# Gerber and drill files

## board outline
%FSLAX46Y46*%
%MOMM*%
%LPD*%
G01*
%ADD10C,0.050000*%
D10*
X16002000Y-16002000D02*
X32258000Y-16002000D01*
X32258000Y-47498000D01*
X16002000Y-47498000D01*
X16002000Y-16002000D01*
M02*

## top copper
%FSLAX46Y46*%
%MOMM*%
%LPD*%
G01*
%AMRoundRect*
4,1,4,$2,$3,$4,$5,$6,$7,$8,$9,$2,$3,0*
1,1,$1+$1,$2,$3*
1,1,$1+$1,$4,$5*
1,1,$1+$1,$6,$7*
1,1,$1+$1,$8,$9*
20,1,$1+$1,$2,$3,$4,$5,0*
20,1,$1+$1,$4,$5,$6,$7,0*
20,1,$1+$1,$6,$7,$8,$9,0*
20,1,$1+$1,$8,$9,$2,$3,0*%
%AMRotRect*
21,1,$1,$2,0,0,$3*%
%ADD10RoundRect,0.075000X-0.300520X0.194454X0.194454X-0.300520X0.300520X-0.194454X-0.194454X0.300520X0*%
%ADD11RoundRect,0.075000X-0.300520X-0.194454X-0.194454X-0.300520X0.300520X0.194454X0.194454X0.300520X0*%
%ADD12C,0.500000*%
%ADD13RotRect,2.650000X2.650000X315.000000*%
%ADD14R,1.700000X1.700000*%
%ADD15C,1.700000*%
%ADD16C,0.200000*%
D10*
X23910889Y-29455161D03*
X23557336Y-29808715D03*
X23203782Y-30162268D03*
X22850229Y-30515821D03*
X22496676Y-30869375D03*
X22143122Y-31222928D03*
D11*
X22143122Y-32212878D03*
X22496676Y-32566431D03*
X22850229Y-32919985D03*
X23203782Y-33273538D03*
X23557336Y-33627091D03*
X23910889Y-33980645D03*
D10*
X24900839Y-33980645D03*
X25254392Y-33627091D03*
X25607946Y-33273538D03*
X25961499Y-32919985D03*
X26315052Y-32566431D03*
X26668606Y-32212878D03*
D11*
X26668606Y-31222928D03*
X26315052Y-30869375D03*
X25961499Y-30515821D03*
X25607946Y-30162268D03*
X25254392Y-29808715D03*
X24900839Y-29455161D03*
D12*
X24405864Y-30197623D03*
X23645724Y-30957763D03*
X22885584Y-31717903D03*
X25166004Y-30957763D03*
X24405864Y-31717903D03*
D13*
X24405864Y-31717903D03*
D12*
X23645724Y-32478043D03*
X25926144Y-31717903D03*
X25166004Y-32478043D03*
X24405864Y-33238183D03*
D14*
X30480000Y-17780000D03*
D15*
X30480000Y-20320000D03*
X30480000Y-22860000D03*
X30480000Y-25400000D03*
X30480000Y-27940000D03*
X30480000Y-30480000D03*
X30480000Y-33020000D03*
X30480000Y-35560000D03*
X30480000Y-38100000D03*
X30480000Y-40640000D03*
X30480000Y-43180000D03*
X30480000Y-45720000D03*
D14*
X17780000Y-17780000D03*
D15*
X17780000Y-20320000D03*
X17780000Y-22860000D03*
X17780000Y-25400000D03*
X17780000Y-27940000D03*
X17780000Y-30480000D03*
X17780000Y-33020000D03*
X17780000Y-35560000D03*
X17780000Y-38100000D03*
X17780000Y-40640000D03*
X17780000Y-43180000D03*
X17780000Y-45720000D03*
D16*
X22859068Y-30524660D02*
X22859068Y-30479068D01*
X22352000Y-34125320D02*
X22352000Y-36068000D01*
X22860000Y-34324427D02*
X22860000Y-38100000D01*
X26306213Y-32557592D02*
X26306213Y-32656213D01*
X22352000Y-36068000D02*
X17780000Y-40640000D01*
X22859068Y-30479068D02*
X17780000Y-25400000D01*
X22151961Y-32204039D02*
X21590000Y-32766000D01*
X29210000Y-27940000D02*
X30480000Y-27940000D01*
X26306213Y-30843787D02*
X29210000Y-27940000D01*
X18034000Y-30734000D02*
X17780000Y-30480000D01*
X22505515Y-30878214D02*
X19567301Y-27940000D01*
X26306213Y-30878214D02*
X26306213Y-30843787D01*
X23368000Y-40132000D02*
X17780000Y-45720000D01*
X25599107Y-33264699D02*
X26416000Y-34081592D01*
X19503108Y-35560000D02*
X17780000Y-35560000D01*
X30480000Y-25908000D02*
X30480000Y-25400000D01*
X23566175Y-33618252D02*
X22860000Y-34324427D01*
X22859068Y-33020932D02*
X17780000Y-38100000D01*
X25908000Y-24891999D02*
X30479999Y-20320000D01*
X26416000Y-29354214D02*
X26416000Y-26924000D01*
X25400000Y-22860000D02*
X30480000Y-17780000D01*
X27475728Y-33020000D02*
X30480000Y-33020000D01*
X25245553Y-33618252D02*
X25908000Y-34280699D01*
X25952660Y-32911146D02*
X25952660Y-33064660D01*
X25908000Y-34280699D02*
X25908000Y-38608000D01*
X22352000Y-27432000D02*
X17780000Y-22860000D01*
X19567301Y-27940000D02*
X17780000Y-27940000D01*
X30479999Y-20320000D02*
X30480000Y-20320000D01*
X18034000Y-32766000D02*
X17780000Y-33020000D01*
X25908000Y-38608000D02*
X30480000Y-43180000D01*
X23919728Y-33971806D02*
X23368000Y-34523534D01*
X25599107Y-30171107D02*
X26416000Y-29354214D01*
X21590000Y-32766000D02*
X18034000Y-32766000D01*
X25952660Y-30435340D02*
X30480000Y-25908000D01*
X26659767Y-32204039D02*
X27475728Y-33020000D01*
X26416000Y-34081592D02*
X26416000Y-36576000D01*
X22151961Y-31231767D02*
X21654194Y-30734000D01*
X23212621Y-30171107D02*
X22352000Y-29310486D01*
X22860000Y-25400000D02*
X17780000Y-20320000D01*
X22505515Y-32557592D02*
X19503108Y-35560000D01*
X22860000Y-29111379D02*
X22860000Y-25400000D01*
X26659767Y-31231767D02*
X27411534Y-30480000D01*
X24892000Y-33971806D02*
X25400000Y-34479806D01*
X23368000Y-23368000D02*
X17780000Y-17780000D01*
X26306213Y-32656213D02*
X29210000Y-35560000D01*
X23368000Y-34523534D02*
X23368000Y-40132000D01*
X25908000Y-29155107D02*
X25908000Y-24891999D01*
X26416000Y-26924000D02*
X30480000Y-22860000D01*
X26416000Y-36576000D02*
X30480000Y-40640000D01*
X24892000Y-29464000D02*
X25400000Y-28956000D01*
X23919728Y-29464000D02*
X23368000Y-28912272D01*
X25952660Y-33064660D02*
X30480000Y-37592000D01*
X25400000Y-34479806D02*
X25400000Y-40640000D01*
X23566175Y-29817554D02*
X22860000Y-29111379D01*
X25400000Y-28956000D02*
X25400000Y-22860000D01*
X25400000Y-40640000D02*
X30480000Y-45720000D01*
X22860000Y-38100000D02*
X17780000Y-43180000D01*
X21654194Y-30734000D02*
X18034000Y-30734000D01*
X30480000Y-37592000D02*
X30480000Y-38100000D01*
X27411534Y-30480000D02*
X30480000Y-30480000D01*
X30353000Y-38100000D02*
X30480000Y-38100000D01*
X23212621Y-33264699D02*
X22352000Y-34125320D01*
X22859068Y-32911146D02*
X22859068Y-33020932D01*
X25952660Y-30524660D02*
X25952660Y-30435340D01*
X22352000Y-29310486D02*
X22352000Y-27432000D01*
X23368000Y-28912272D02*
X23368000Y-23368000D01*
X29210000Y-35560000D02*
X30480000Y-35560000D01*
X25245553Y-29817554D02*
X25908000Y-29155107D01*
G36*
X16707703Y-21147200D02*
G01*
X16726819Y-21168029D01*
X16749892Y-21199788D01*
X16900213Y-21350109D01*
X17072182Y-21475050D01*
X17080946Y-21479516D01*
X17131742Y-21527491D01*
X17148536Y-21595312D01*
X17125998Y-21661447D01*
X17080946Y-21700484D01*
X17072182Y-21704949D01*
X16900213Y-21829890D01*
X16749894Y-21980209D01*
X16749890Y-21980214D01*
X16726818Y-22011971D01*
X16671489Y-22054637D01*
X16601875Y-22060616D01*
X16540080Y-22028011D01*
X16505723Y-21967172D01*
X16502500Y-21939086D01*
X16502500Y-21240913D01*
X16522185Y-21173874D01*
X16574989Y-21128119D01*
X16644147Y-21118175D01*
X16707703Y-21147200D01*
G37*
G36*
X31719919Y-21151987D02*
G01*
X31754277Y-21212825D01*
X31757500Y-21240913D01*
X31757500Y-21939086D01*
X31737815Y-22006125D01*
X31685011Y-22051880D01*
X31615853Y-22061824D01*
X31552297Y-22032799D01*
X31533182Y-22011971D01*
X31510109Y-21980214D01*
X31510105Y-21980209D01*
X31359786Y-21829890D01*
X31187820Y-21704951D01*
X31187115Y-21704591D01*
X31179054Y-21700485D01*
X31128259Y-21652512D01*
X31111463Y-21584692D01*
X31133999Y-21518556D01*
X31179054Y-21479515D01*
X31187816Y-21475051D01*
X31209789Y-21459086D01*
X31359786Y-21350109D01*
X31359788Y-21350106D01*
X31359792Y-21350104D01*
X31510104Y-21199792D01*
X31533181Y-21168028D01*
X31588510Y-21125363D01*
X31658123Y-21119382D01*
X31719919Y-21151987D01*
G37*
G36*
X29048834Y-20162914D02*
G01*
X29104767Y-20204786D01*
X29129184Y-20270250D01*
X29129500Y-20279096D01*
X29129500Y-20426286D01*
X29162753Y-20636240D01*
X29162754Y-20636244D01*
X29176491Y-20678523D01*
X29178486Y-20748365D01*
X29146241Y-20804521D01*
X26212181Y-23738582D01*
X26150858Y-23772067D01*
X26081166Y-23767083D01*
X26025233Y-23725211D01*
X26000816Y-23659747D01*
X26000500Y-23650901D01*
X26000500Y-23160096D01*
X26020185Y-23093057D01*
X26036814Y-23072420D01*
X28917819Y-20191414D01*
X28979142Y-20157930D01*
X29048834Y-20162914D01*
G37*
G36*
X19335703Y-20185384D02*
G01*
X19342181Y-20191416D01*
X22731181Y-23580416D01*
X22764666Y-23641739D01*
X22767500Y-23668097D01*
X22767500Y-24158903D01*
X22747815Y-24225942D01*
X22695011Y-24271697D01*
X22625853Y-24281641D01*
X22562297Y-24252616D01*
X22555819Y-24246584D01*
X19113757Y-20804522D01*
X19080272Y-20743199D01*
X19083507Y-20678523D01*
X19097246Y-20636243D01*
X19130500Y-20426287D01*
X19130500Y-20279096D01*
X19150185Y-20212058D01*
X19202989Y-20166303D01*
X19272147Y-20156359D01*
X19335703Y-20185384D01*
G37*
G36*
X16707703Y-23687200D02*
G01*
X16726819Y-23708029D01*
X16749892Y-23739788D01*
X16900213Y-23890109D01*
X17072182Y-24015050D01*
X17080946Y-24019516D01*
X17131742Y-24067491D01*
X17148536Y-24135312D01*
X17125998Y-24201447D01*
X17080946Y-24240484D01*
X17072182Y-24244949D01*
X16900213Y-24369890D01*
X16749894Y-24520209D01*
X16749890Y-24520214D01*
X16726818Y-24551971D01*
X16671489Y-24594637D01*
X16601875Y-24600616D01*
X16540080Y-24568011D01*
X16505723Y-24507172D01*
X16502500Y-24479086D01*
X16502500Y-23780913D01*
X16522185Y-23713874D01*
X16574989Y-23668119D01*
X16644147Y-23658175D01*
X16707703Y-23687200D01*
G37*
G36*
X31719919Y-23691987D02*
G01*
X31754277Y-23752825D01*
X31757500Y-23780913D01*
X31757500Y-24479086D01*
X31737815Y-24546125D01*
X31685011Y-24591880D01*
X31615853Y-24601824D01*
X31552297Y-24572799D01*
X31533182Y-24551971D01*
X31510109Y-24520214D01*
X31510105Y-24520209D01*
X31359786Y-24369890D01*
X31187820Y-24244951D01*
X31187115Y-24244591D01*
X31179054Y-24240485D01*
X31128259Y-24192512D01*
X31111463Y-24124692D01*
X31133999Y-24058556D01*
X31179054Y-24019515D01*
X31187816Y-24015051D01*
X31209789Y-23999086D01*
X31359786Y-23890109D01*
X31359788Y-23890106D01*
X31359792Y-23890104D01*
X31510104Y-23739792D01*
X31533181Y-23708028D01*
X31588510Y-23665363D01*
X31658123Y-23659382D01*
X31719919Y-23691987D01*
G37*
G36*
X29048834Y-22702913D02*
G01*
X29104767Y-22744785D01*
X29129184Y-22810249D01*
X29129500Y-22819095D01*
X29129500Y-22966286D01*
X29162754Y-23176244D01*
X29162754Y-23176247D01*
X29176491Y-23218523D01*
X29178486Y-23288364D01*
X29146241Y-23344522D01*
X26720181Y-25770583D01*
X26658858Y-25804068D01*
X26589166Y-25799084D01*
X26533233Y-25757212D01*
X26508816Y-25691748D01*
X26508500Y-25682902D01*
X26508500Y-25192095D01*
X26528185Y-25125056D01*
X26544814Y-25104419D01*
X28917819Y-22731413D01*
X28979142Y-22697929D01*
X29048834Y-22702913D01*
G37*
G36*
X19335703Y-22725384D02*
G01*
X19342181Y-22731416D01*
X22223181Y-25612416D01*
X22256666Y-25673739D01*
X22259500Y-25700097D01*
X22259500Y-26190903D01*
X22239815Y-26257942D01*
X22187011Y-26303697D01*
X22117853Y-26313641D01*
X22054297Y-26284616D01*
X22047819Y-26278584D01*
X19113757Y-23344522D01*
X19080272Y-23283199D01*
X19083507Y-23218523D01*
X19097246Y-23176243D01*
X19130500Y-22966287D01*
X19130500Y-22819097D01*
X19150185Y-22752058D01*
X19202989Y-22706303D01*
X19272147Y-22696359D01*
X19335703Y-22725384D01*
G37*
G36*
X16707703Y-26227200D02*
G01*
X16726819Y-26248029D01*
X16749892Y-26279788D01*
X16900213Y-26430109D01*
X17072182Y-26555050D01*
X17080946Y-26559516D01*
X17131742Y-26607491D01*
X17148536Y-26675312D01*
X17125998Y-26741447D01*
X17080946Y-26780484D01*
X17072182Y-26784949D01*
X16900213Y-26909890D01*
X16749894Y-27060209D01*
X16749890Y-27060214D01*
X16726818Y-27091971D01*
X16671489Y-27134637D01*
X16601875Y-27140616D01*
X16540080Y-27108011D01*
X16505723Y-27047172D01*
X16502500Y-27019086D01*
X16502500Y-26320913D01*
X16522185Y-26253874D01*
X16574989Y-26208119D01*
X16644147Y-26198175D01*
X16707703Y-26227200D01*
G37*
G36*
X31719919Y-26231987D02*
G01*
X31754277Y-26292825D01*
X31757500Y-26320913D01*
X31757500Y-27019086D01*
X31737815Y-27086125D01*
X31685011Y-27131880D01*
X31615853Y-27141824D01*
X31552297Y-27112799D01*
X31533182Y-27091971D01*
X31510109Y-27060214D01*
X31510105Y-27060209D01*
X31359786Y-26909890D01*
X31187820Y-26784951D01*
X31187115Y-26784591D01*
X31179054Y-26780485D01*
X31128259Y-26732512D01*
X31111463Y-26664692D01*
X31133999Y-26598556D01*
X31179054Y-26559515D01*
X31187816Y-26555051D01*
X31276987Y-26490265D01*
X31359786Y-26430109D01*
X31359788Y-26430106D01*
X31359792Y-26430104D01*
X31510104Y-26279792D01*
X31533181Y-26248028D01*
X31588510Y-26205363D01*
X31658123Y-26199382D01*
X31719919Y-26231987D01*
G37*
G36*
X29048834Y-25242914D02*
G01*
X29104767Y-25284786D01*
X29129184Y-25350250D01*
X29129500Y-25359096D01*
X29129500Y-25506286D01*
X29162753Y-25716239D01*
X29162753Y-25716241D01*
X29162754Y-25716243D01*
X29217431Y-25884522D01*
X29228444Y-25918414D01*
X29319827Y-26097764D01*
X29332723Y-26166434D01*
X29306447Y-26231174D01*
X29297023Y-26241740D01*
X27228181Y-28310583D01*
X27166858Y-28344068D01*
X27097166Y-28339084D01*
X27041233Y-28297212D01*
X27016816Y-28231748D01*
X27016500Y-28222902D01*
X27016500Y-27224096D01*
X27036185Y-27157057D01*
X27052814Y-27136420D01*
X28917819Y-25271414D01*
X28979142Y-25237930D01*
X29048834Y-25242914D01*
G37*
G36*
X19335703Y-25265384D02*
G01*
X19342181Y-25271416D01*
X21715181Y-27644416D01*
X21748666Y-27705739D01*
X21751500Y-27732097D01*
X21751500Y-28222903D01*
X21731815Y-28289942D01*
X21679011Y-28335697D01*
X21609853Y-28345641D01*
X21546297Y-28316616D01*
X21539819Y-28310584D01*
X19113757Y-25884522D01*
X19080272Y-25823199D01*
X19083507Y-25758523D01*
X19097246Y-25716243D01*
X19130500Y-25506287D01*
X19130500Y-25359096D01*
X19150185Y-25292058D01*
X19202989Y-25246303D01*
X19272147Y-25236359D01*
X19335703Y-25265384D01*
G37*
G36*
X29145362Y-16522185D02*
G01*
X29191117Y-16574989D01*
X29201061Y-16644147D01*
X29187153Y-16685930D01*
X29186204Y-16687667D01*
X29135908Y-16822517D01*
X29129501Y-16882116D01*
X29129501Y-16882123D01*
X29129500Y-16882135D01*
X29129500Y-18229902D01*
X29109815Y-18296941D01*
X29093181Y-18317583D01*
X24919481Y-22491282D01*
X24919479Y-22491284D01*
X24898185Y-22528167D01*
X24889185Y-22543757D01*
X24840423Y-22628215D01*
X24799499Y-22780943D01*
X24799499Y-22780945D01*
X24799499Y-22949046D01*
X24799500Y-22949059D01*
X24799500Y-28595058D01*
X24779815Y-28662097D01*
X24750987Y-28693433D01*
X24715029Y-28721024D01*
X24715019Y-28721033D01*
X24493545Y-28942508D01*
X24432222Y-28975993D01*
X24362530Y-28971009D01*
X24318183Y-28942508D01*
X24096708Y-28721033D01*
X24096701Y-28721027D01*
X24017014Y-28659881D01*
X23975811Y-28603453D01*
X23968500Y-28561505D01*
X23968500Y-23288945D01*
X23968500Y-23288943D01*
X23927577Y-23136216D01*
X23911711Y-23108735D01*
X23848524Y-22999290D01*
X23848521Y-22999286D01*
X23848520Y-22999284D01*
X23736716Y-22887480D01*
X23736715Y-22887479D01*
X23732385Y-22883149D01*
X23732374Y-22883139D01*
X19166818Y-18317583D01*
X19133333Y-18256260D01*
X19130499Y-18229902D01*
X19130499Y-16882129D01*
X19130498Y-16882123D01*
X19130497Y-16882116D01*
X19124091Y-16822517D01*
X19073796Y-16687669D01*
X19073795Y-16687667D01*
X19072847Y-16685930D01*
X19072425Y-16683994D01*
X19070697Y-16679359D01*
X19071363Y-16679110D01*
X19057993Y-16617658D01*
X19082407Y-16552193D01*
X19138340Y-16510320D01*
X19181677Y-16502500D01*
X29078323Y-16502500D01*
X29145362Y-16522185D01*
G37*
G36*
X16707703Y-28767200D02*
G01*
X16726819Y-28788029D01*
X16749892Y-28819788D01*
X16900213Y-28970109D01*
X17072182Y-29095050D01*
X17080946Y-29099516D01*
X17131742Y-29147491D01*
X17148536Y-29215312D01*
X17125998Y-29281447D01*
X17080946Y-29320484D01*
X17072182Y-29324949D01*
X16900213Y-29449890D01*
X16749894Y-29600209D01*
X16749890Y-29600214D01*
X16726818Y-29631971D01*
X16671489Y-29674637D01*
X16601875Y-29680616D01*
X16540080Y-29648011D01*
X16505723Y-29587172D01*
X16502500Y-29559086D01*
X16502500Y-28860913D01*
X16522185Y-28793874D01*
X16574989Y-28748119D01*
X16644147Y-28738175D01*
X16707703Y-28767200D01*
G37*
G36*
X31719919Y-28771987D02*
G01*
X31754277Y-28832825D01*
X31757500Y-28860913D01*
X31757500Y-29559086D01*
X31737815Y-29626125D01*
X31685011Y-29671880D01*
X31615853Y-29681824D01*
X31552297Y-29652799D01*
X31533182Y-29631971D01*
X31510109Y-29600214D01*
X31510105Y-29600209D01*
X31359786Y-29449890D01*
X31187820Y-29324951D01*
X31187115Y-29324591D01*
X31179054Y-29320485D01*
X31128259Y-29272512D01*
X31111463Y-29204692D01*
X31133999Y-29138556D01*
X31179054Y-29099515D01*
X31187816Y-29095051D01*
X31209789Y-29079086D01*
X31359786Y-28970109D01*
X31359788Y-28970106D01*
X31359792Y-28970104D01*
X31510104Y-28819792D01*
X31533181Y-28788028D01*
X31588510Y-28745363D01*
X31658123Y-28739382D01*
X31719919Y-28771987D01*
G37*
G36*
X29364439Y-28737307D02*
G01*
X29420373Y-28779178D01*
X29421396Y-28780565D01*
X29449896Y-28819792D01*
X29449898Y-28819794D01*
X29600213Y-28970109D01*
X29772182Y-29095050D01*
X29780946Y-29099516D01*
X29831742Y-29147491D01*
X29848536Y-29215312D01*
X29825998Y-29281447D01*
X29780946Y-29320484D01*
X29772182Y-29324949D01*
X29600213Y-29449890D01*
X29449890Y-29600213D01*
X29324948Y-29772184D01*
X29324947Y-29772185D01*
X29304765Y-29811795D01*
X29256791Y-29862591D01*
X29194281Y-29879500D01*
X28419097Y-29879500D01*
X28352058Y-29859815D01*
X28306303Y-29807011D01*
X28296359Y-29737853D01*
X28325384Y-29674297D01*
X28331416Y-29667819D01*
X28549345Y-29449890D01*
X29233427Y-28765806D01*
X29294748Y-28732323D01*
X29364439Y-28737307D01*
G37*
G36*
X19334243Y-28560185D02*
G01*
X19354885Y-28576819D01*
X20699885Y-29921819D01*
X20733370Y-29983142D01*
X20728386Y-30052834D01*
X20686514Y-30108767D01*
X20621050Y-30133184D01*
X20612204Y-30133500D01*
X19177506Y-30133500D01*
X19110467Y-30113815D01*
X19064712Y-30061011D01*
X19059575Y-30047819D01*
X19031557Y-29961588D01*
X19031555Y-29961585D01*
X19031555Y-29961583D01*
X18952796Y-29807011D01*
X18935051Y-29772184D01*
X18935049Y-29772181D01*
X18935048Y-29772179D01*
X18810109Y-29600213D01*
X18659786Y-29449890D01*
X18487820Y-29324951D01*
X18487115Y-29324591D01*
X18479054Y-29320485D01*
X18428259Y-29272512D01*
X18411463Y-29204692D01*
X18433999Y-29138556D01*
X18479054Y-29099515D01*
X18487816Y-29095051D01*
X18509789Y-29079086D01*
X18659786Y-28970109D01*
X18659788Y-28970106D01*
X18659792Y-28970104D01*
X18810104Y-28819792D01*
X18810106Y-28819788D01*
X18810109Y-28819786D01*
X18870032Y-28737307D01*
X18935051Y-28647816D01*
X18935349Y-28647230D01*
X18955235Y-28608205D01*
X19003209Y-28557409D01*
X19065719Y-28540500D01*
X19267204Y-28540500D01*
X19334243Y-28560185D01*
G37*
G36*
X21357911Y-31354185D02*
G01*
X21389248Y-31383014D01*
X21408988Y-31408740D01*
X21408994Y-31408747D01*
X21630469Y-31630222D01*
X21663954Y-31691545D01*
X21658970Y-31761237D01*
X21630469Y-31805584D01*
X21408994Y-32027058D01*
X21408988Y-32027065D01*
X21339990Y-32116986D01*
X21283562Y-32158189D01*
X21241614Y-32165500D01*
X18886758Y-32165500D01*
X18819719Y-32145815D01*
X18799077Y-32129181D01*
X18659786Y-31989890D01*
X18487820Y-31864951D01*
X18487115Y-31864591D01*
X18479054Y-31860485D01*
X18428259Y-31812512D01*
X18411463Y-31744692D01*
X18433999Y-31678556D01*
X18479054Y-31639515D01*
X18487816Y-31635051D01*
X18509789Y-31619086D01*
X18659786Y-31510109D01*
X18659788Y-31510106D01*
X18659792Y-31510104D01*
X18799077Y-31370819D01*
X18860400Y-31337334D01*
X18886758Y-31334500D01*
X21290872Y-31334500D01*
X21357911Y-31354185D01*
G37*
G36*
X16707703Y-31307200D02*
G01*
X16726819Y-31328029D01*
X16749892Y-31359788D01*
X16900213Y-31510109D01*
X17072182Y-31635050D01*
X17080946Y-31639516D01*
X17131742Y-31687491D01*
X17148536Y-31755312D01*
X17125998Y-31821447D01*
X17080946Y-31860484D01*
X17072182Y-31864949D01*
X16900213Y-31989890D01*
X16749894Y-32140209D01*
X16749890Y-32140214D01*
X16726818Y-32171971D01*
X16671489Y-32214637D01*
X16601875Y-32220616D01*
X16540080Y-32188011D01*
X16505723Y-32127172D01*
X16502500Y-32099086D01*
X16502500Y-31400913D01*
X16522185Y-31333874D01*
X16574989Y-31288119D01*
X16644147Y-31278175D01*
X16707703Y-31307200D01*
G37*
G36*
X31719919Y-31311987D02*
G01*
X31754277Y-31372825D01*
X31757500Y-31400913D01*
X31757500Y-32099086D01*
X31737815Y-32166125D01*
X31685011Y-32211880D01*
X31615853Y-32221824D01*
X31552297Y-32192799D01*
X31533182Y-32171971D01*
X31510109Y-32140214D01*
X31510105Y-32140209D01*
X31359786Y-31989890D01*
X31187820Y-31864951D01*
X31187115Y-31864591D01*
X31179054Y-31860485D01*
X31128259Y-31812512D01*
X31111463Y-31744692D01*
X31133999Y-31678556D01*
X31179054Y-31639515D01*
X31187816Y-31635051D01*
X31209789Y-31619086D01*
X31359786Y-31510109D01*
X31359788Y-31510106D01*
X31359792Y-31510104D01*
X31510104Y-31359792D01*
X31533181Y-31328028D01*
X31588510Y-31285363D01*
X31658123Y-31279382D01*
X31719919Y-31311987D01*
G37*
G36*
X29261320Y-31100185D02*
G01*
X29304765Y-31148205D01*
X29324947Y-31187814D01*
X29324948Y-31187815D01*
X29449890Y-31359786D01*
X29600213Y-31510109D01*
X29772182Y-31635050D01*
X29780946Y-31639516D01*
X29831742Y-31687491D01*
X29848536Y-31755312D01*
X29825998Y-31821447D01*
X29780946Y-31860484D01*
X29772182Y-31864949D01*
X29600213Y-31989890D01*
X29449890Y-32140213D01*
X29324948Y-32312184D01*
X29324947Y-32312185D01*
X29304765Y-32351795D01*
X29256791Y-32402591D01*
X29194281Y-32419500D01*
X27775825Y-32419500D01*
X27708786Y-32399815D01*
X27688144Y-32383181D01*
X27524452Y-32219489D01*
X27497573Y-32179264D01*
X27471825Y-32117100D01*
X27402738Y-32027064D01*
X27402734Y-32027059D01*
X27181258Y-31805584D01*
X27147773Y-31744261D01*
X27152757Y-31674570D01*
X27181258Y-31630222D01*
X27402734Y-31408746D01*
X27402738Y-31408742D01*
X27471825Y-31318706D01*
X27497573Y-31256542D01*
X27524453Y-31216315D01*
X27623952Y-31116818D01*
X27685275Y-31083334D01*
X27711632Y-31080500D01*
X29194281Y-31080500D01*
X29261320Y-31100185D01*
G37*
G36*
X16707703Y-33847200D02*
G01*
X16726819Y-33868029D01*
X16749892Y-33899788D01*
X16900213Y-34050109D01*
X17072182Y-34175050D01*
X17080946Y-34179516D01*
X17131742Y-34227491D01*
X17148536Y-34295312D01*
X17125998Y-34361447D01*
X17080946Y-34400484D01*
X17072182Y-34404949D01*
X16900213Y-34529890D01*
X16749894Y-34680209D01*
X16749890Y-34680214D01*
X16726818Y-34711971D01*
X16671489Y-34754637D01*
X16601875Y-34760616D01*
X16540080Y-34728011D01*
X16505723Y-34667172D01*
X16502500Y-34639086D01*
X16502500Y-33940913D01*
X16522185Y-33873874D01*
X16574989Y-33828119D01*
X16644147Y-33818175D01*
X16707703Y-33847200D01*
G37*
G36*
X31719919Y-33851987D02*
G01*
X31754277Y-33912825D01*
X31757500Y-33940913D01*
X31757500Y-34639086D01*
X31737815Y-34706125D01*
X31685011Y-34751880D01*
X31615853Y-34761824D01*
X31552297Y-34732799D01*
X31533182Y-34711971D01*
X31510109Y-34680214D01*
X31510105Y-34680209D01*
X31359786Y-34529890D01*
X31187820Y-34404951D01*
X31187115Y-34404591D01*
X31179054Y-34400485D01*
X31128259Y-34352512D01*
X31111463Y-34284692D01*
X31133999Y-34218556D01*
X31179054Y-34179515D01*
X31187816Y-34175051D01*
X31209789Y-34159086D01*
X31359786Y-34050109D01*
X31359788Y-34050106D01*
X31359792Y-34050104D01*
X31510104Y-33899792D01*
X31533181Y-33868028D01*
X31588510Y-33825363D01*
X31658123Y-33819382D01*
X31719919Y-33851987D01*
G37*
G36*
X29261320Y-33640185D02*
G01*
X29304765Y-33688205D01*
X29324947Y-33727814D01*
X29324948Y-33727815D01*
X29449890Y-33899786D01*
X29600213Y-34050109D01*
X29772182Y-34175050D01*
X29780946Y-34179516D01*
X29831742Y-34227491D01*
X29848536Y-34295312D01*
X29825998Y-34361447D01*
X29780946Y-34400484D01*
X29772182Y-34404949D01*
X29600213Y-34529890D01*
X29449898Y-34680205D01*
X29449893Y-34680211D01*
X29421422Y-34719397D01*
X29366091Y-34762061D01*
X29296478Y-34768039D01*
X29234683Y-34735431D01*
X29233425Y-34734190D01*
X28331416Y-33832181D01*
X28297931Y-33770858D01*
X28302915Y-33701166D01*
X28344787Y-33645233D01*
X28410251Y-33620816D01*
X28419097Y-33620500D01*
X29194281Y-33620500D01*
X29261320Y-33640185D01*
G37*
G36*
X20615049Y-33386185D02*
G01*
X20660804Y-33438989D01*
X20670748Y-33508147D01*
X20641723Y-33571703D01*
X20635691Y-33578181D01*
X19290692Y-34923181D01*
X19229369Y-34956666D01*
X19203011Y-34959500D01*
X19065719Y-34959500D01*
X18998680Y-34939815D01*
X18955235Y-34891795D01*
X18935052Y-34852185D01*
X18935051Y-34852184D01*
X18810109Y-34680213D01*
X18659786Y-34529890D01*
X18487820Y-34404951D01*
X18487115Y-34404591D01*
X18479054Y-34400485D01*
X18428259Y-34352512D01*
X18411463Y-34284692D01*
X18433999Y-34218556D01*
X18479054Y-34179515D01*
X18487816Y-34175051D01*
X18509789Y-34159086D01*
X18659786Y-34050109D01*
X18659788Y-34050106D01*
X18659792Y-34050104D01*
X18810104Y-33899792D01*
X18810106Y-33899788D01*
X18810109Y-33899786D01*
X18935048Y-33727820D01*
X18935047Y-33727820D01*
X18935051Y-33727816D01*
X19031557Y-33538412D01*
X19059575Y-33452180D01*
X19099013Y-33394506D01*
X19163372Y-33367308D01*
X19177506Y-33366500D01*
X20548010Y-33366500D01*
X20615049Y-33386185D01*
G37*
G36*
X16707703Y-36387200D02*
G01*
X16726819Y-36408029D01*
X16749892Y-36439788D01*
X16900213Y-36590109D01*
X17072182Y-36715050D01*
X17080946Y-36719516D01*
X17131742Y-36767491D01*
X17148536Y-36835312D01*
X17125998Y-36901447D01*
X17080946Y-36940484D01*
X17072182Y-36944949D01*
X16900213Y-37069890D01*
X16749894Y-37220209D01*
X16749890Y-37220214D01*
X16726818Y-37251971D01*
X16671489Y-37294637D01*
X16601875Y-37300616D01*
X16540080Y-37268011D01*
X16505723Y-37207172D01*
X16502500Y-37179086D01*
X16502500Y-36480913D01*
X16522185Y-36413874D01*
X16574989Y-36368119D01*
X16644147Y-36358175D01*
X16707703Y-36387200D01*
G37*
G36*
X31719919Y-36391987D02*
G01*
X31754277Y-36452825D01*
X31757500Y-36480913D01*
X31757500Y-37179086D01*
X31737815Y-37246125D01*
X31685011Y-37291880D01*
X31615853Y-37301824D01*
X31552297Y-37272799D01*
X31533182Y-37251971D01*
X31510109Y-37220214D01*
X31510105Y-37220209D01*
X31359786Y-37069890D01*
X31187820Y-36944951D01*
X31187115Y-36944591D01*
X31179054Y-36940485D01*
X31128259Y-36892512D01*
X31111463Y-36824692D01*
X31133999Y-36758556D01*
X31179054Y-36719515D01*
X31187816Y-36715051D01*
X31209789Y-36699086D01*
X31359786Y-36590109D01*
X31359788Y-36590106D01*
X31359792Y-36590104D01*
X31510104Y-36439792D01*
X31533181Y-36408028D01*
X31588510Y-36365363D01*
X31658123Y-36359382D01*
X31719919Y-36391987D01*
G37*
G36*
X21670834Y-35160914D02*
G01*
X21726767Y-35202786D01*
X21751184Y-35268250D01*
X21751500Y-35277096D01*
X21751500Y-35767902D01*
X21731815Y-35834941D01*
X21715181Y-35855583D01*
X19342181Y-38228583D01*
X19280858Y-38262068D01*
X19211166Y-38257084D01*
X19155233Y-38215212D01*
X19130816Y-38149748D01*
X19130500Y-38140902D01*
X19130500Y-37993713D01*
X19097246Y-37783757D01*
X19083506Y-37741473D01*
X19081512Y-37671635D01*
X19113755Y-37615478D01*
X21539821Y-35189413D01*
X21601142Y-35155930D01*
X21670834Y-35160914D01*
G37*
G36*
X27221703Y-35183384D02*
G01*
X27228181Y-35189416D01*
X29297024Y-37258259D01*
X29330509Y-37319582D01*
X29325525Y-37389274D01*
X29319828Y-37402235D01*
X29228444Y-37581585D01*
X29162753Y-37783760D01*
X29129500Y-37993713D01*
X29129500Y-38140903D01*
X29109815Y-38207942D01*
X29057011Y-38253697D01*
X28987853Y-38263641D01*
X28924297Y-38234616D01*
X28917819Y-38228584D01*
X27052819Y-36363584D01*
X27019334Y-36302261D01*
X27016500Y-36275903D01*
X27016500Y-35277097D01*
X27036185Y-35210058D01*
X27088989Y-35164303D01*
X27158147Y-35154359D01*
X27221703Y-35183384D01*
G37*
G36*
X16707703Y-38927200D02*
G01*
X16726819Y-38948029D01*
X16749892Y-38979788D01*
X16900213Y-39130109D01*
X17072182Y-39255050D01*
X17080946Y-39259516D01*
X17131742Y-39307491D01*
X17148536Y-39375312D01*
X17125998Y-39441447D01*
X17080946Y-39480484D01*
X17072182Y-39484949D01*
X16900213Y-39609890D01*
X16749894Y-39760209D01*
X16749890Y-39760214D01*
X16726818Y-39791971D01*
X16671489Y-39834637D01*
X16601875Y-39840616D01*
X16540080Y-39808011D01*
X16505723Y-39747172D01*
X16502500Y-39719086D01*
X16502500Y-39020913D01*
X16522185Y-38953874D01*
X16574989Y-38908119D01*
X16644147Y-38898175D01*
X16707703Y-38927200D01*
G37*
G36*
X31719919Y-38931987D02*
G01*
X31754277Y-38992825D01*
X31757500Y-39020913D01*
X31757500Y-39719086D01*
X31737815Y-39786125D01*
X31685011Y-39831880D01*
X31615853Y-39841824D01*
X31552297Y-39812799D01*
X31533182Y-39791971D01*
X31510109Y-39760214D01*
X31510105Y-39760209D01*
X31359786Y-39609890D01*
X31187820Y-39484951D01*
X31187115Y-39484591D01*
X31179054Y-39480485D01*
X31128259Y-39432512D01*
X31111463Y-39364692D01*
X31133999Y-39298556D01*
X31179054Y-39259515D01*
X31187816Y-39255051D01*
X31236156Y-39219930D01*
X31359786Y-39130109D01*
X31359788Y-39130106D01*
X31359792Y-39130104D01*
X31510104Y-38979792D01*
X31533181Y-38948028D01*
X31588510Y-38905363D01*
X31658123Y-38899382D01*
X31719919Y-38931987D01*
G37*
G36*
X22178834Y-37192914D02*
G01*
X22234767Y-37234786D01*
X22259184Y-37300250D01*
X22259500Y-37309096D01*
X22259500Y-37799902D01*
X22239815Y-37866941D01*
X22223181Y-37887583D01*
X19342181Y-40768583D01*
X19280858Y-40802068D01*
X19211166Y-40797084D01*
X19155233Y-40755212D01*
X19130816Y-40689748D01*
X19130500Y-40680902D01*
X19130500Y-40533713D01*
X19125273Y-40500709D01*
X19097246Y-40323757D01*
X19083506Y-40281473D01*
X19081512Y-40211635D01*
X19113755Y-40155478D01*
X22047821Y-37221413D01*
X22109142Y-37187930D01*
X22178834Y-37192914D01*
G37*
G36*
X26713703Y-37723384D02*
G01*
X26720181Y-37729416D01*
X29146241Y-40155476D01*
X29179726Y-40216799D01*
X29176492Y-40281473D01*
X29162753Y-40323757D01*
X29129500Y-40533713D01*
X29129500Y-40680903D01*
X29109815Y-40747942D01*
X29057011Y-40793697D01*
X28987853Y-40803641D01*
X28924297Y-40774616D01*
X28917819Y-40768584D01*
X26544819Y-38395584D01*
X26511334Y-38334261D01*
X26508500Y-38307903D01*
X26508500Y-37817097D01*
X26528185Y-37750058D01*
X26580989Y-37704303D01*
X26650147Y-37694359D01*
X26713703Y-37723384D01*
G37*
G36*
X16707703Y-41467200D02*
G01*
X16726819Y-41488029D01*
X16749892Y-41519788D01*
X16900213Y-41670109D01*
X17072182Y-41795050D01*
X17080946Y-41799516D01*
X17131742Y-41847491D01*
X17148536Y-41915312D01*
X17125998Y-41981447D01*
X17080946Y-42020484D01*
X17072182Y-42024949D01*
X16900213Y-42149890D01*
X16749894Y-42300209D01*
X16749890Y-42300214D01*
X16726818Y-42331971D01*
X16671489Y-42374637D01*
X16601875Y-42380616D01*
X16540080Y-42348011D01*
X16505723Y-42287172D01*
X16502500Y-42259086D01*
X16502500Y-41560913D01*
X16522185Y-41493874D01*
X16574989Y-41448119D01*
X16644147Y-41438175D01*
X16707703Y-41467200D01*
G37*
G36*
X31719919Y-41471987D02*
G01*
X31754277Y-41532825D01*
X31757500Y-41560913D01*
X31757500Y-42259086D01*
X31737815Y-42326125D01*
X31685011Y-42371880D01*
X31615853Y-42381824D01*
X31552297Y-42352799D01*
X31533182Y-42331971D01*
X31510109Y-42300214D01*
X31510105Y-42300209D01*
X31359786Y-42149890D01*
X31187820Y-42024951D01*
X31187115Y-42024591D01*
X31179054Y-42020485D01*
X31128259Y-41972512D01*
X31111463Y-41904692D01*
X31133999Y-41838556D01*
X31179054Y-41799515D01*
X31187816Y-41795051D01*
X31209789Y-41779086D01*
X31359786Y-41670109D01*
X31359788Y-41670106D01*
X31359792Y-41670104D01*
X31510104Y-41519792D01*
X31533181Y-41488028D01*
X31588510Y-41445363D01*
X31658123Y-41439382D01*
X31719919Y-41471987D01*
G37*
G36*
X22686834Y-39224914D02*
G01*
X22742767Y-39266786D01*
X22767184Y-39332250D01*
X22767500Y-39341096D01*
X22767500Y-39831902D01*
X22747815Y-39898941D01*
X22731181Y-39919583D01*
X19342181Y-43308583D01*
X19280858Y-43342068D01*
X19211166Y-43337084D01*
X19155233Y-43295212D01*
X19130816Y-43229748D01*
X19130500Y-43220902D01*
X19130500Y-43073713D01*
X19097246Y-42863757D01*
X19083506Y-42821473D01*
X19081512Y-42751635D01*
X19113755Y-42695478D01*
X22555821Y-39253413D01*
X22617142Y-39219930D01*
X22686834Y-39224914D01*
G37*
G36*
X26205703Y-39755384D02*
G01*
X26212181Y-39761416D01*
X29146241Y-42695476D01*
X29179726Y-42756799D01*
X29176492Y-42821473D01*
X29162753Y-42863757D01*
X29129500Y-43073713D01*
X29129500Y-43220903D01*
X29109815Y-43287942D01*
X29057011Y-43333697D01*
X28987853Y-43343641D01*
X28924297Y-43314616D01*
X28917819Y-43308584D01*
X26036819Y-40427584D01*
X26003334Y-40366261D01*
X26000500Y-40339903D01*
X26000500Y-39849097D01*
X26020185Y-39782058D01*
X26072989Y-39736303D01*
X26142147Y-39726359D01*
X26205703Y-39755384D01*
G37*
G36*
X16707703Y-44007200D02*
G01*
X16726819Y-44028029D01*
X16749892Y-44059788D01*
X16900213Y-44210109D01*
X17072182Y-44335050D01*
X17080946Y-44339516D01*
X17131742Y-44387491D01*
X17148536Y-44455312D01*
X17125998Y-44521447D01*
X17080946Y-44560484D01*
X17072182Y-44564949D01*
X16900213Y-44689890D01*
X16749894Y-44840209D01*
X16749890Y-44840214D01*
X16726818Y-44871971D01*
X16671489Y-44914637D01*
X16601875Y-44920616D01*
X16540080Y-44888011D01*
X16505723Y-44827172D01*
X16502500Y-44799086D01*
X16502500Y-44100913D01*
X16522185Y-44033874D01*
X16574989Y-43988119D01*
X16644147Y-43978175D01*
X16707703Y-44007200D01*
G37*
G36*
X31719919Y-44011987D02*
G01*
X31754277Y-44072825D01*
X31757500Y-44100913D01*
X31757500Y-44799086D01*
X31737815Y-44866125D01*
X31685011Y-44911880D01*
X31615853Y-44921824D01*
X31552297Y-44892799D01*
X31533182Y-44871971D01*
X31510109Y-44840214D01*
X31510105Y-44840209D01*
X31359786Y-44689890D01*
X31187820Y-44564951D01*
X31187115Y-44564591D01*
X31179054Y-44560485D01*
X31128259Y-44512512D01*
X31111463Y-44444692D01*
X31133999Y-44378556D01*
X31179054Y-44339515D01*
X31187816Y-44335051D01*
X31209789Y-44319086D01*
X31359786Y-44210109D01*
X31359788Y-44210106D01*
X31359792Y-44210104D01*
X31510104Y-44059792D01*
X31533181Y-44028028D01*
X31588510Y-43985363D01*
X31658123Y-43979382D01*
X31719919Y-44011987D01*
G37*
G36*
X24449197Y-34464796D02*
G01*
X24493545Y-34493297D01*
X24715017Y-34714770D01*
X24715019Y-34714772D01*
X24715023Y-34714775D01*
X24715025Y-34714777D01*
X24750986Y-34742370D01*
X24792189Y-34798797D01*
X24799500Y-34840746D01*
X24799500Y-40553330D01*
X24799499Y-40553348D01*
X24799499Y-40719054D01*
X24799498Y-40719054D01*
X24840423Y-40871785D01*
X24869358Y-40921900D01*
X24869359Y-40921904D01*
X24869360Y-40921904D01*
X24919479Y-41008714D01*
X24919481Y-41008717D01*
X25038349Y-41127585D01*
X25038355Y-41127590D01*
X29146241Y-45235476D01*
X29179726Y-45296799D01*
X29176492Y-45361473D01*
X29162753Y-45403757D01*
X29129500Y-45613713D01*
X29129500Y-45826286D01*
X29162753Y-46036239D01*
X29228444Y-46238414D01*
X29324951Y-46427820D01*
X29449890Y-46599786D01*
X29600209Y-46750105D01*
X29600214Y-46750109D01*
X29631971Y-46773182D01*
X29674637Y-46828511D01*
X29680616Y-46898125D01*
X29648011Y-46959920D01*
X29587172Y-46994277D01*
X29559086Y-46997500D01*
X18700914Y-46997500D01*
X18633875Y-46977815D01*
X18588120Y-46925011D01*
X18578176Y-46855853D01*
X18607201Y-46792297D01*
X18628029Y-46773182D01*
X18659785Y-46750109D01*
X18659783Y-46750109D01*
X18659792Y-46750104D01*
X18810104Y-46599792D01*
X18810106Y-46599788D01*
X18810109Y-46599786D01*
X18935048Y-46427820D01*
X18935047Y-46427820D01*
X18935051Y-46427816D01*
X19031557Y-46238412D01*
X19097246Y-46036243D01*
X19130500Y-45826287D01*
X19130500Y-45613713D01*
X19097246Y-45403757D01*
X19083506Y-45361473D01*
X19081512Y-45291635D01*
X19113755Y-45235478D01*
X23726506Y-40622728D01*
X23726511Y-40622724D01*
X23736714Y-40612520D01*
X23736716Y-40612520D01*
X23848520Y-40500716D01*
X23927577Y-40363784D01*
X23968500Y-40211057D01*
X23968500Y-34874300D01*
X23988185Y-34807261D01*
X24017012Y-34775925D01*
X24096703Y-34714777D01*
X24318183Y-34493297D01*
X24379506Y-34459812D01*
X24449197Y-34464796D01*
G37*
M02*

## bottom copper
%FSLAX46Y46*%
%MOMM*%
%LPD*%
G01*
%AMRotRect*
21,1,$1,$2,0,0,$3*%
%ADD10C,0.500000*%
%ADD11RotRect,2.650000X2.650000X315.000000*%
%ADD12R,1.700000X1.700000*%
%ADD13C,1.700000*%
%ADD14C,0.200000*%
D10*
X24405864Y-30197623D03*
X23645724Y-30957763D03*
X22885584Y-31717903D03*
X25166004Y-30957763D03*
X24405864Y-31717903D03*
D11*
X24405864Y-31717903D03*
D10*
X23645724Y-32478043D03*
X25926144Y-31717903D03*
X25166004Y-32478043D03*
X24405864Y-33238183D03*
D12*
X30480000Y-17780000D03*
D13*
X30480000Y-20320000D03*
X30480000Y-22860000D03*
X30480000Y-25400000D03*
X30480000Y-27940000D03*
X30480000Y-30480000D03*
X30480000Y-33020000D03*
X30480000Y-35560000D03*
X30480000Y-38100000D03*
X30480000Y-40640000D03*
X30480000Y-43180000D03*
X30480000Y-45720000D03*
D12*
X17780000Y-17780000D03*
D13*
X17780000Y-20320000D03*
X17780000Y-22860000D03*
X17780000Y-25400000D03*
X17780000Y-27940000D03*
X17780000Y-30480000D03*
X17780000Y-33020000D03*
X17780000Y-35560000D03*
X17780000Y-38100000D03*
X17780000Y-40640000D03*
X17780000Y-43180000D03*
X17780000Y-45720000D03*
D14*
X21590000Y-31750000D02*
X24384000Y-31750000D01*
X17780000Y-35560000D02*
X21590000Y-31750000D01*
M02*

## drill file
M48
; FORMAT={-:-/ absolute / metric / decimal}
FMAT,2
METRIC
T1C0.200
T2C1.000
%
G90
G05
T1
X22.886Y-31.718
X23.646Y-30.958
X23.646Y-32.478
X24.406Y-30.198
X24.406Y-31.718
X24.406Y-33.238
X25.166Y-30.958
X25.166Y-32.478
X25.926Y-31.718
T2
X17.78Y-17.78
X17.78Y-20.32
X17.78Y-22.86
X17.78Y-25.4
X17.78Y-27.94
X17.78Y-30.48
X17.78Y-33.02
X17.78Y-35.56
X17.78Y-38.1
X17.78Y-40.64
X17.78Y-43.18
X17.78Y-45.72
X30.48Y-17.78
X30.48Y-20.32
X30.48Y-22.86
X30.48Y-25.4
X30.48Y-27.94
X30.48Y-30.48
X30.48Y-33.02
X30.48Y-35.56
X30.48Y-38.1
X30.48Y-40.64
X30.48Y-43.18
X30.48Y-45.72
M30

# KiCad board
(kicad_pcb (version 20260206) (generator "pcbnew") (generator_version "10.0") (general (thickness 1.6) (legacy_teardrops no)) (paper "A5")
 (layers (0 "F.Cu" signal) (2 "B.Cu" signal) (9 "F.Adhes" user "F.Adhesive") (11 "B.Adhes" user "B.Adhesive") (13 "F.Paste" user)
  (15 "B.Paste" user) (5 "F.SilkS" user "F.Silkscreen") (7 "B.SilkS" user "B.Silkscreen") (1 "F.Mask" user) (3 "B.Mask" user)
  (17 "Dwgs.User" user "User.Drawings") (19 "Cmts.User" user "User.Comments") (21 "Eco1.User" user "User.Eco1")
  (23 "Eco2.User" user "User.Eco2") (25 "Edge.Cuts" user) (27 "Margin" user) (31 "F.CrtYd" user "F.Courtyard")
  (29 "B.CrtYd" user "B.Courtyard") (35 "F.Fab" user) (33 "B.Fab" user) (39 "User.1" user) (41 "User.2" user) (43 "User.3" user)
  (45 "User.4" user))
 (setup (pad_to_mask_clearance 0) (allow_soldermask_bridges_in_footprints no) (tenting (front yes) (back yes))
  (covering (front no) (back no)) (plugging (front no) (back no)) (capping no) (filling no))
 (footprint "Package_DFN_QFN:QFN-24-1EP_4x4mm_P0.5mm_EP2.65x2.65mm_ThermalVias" (layer "F.Cu") (at 24.405864 31.717903 -45)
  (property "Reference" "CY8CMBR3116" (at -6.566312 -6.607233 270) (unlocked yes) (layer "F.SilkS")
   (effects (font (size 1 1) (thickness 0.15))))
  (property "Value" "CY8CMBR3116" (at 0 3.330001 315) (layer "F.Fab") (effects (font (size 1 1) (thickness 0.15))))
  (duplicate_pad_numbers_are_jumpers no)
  (pad "" smd roundrect (at -0.66 -0.66 315) (size 1.15 1.15) (layers "F.Paste") (roundrect_rratio 0.217391))
  (pad "" smd roundrect (at -0.66 0.66 315) (size 1.15 1.15) (layers "F.Paste") (roundrect_rratio 0.217391))
  (pad "" smd roundrect (at 0.66 -0.66 315) (size 1.15 1.15) (layers "F.Paste") (roundrect_rratio 0.217391))
  (pad "" smd roundrect (at 0.66 0.66 315) (size 1.15 1.15) (layers "F.Paste") (roundrect_rratio 0.217391))
  (pad "1" smd roundrect (at -1.95 -1.25 315) (size 0.85 0.3) (layers "F.Cu" "F.Mask" "F.Paste") (roundrect_rratio 0.25) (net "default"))
  (pad "2" smd roundrect (at -1.95 -0.75 315) (size 0.85 0.3) (layers "F.Cu" "F.Mask" "F.Paste") (roundrect_rratio 0.25) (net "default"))
  (pad "3" smd roundrect (at -1.95 -0.25 315) (size 0.85 0.3) (layers "F.Cu" "F.Mask" "F.Paste") (roundrect_rratio 0.25) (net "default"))
  (pad "4" smd roundrect (at -1.95 0.25 315) (size 0.85 0.3) (layers "F.Cu" "F.Mask" "F.Paste") (roundrect_rratio 0.25) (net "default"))
  (pad "5" smd roundrect (at -1.95 0.75 315) (size 0.85 0.3) (layers "F.Cu" "F.Mask" "F.Paste") (roundrect_rratio 0.25) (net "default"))
  (pad "6" smd roundrect (at -1.95 1.25 315) (size 0.85 0.3) (layers "F.Cu" "F.Mask" "F.Paste") (roundrect_rratio 0.25) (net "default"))
  (pad "7" smd roundrect (at -1.25 1.95 315) (size 0.3 0.85) (layers "F.Cu" "F.Mask" "F.Paste") (roundrect_rratio 0.25) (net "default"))
  (pad "8" smd roundrect (at -0.75 1.95 315) (size 0.3 0.85) (layers "F.Cu" "F.Mask" "F.Paste") (roundrect_rratio 0.25) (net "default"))
  (pad "9" smd roundrect (at -0.25 1.95 315) (size 0.3 0.85) (layers "F.Cu" "F.Mask" "F.Paste") (roundrect_rratio 0.25) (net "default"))
  (pad "10" smd roundrect (at 0.25 1.95 315) (size 0.3 0.85) (layers "F.Cu" "F.Mask" "F.Paste") (roundrect_rratio 0.25) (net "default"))
  (pad "11" smd roundrect (at 0.75 1.95 315) (size 0.3 0.85) (layers "F.Cu" "F.Mask" "F.Paste") (roundrect_rratio 0.25) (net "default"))
  (pad "12" smd roundrect (at 1.25 1.95 315) (size 0.3 0.85) (layers "F.Cu" "F.Mask" "F.Paste") (roundrect_rratio 0.25) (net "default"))
  (pad "13" smd roundrect (at 1.95 1.25 315) (size 0.85 0.3) (layers "F.Cu" "F.Mask" "F.Paste") (roundrect_rratio 0.25) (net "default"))
  (pad "14" smd roundrect (at 1.95 0.75 315) (size 0.85 0.3) (layers "F.Cu" "F.Mask" "F.Paste") (roundrect_rratio 0.25) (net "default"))
  (pad "15" smd roundrect (at 1.95 0.25 315) (size 0.85 0.3) (layers "F.Cu" "F.Mask" "F.Paste") (roundrect_rratio 0.25) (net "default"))
  (pad "16" smd roundrect (at 1.95 -0.25 315) (size 0.85 0.3) (layers "F.Cu" "F.Mask" "F.Paste") (roundrect_rratio 0.25) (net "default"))
  (pad "17" smd roundrect (at 1.95 -0.75 315) (size 0.85 0.3) (layers "F.Cu" "F.Mask" "F.Paste") (roundrect_rratio 0.25) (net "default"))
  (pad "18" smd roundrect (at 1.95 -1.25 315) (size 0.85 0.3) (layers "F.Cu" "F.Mask" "F.Paste") (roundrect_rratio 0.25) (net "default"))
  (pad "19" smd roundrect (at 1.25 -1.95 315) (size 0.3 0.85) (layers "F.Cu" "F.Mask" "F.Paste") (roundrect_rratio 0.25) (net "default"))
  (pad "20" smd roundrect (at 0.75 -1.95 315) (size 0.3 0.85) (layers "F.Cu" "F.Mask" "F.Paste") (roundrect_rratio 0.25) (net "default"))
  (pad "21" smd roundrect (at 0.25 -1.95 315) (size 0.3 0.85) (layers "F.Cu" "F.Mask" "F.Paste") (roundrect_rratio 0.25) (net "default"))
  (pad "22" smd roundrect (at -0.25 -1.95 315) (size 0.3 0.85) (layers "F.Cu" "F.Mask" "F.Paste") (roundrect_rratio 0.25) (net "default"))
  (pad "23" smd roundrect (at -0.75 -1.95 315) (size 0.3 0.85) (layers "F.Cu" "F.Mask" "F.Paste") (roundrect_rratio 0.25) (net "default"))
  (pad "24" smd roundrect (at -1.25 -1.95 315) (size 0.3 0.85) (layers "F.Cu" "F.Mask" "F.Paste") (roundrect_rratio 0.25) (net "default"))
  (pad "25" thru_hole circle (at -1.075 -1.075 315) (size 0.5 0.5) (drill 0.2) (layers "*.Cu") (remove_unused_layers no))
  (pad "25" thru_hole circle (at -1.075 0 315) (size 0.5 0.5) (drill 0.2) (layers "*.Cu") (remove_unused_layers no))
  (pad "25" thru_hole circle (at -1.075 1.075 315) (size 0.5 0.5) (drill 0.2) (layers "*.Cu") (remove_unused_layers no))
  (pad "25" thru_hole circle (at 0 -1.075 315) (size 0.5 0.5) (drill 0.2) (layers "*.Cu") (remove_unused_layers no))
  (pad "25" thru_hole circle (at 0 0 315) (size 0.5 0.5) (drill 0.2) (layers "*.Cu") (remove_unused_layers no))
  (pad "25" smd rect (at 0 0 315) (size 2.65 2.65) (layers "F.Cu" "F.Mask") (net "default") (zone_connect 2))
  (pad "25" smd rect (at 0 0 315) (size 2.65 2.65) (layers "B.Cu") (zone_connect 2))
  (pad "25" thru_hole circle (at 0 1.075 315) (size 0.5 0.5) (drill 0.2) (layers "*.Cu") (remove_unused_layers no))
  (pad "25" thru_hole circle (at 1.075 -1.075 315) (size 0.5 0.5) (drill 0.2) (layers "*.Cu") (remove_unused_layers no))
  (pad "25" thru_hole circle (at 1.075 0 315) (size 0.5 0.5) (drill 0.2) (layers "*.Cu") (remove_unused_layers no))
  (pad "25" thru_hole circle (at 1.075 1.075 315) (size 0.5 0.5) (drill 0.2) (layers "*.Cu") (remove_unused_layers no)))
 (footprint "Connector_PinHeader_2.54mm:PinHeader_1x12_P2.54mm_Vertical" (layer "B.Cu") (at 30.48 17.78 180)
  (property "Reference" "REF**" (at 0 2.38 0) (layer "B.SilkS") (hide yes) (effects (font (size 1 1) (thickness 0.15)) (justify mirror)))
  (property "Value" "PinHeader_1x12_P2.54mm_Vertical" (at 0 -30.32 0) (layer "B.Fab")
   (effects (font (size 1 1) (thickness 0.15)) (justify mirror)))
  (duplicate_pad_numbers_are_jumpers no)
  (pad "1" thru_hole rect (at 0 0 180) (size 1.7 1.7) (drill 1) (layers "*.Cu" "*.Mask") (remove_unused_layers no) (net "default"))
  (pad "2" thru_hole circle (at 0 -2.54 180) (size 1.7 1.7) (drill 1) (layers "*.Cu" "*.Mask") (remove_unused_layers no) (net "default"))
  (pad "3" thru_hole circle (at 0 -5.08 180) (size 1.7 1.7) (drill 1) (layers "*.Cu" "*.Mask") (remove_unused_layers no) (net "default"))
  (pad "4" thru_hole circle (at 0 -7.62 180) (size 1.7 1.7) (drill 1) (layers "*.Cu" "*.Mask") (remove_unused_layers no) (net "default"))
  (pad "5" thru_hole circle (at 0 -10.16 180) (size 1.7 1.7) (drill 1) (layers "*.Cu" "*.Mask") (remove_unused_layers no) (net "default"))
  (pad "6" thru_hole circle (at 0 -12.7 180) (size 1.7 1.7) (drill 1) (layers "*.Cu" "*.Mask") (remove_unused_layers no) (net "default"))
  (pad "7" thru_hole circle (at 0 -15.24 180) (size 1.7 1.7) (drill 1) (layers "*.Cu" "*.Mask") (remove_unused_layers no) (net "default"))
  (pad "8" thru_hole circle (at 0 -17.78 180) (size 1.7 1.7) (drill 1) (layers "*.Cu" "*.Mask") (remove_unused_layers no) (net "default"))
  (pad "9" thru_hole circle (at 0 -20.32 180) (size 1.7 1.7) (drill 1) (layers "*.Cu" "*.Mask") (remove_unused_layers no) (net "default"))
  (pad "10" thru_hole circle (at 0 -22.86 180) (size 1.7 1.7) (drill 1) (layers "*.Cu" "*.Mask") (remove_unused_layers no) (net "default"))
  (pad "11" thru_hole circle (at 0 -25.4 180) (size 1.7 1.7) (drill 1) (layers "*.Cu" "*.Mask") (remove_unused_layers no) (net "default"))
  (pad "12" thru_hole circle (at 0 -27.94 180) (size 1.7 1.7) (drill 1) (layers "*.Cu" "*.Mask") (remove_unused_layers no) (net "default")))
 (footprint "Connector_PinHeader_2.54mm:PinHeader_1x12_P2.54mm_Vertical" (layer "B.Cu") (at 17.78 17.78 180)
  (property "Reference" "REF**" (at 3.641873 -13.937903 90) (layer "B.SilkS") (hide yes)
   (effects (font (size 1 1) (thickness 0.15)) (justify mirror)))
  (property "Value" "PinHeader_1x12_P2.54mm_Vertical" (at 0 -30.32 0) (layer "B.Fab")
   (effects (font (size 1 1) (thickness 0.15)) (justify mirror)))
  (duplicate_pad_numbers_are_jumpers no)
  (pad "1" thru_hole rect (at 0 0 180) (size 1.7 1.7) (drill 1) (layers "*.Cu" "*.Mask") (remove_unused_layers no) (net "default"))
  (pad "2" thru_hole circle (at 0 -2.54 180) (size 1.7 1.7) (drill 1) (layers "*.Cu" "*.Mask") (remove_unused_layers no) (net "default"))
  (pad "3" thru_hole circle (at 0 -5.08 180) (size 1.7 1.7) (drill 1) (layers "*.Cu" "*.Mask") (remove_unused_layers no) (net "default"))
  (pad "4" thru_hole circle (at 0 -7.62 180) (size 1.7 1.7) (drill 1) (layers "*.Cu" "*.Mask") (remove_unused_layers no) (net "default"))
  (pad "5" thru_hole circle (at 0 -10.16 180) (size 1.7 1.7) (drill 1) (layers "*.Cu" "*.Mask") (remove_unused_layers no) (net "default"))
  (pad "6" thru_hole circle (at 0 -12.7 180) (size 1.7 1.7) (drill 1) (layers "*.Cu" "*.Mask") (remove_unused_layers no) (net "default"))
  (pad "7" thru_hole circle (at 0 -15.24 180) (size 1.7 1.7) (drill 1) (layers "*.Cu" "*.Mask") (remove_unused_layers no) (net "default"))
  (pad "8" thru_hole circle (at 0 -17.78 180) (size 1.7 1.7) (drill 1) (layers "*.Cu" "*.Mask") (remove_unused_layers no) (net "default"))
  (pad "9" thru_hole circle (at 0 -20.32 180) (size 1.7 1.7) (drill 1) (layers "*.Cu" "*.Mask") (remove_unused_layers no) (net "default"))
  (pad "10" thru_hole circle (at 0 -22.86 180) (size 1.7 1.7) (drill 1) (layers "*.Cu" "*.Mask") (remove_unused_layers no) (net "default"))
  (pad "11" thru_hole circle (at 0 -25.4 180) (size 1.7 1.7) (drill 1) (layers "*.Cu" "*.Mask") (remove_unused_layers no) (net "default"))
  (pad "12" thru_hole circle (at 0 -27.94 180) (size 1.7 1.7) (drill 1) (layers "*.Cu" "*.Mask") (remove_unused_layers no) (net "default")))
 (gr_rect (start 16.002 16.002) (end 32.258 47.498) (stroke (width 0.05) (type default)) (fill no) (layer "Edge.Cuts"))
 (segment (start 22.859068 30.52466) (end 22.859068 30.479068) (width 0.2) (layer "F.Cu") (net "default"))
 (segment (start 22.352 34.12532) (end 22.352 36.068) (width 0.2) (layer "F.Cu") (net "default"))
 (segment (start 22.86 34.324427) (end 22.86 38.1) (width 0.2) (layer "F.Cu") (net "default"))
 (segment (start 26.306213 32.557592) (end 26.306213 32.656213) (width 0.2) (layer "F.Cu") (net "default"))
 (segment (start 22.352 36.068) (end 17.78 40.64) (width 0.2) (layer "F.Cu") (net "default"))
 (segment (start 22.859068 30.479068) (end 17.78 25.4) (width 0.2) (layer "F.Cu") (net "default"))
 (segment (start 22.151961 32.204039) (end 21.59 32.766) (width 0.2) (layer "F.Cu") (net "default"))
 (segment (start 29.21 27.94) (end 30.48 27.94) (width 0.2) (layer "F.Cu") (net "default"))
 (segment (start 26.306213 30.843787) (end 29.21 27.94) (width 0.2) (layer "F.Cu") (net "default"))
 (segment (start 18.034 30.734) (end 17.78 30.48) (width 0.2) (layer "F.Cu") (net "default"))
 (segment (start 22.505515 30.878214) (end 19.567301 27.94) (width 0.2) (layer "F.Cu") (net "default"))
 (segment (start 26.306213 30.878214) (end 26.306213 30.843787) (width 0.2) (layer "F.Cu") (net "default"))
 (segment (start 23.368 40.132) (end 17.78 45.72) (width 0.2) (layer "F.Cu") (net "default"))
 (segment (start 25.599107 33.264699) (end 26.416 34.081592) (width 0.2) (layer "F.Cu") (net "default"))
 (segment (start 19.503108 35.56) (end 17.78 35.56) (width 0.2) (layer "F.Cu") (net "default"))
 (segment (start 30.48 25.908) (end 30.48 25.4) (width 0.2) (layer "F.Cu") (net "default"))
 (segment (start 23.566175 33.618252) (end 22.86 34.324427) (width 0.2) (layer "F.Cu") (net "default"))
 (segment (start 22.859068 33.020932) (end 17.78 38.1) (width 0.2) (layer "F.Cu") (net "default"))
 (segment (start 25.908 24.891999) (end 30.479999 20.32) (width 0.2) (layer "F.Cu") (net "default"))
 (segment (start 26.416 29.354214) (end 26.416 26.924) (width 0.2) (layer "F.Cu") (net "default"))
 (segment (start 25.4 22.86) (end 30.48 17.78) (width 0.2) (layer "F.Cu") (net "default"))
 (segment (start 27.475728 33.02) (end 30.48 33.02) (width 0.2) (layer "F.Cu") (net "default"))
 (segment (start 25.245553 33.618252) (end 25.908 34.280699) (width 0.2) (layer "F.Cu") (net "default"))
 (segment (start 25.95266 32.911146) (end 25.95266 33.06466) (width 0.2) (layer "F.Cu") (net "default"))
 (segment (start 25.908 34.280699) (end 25.908 38.608) (width 0.2) (layer "F.Cu") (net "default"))
 (segment (start 22.352 27.432) (end 17.78 22.86) (width 0.2) (layer "F.Cu") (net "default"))
 (segment (start 19.567301 27.94) (end 17.78 27.94) (width 0.2) (layer "F.Cu") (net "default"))
 (segment (start 30.479999 20.32) (end 30.48 20.32) (width 0.2) (layer "F.Cu") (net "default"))
 (segment (start 18.034 32.766) (end 17.78 33.02) (width 0.2) (layer "F.Cu") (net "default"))
 (segment (start 25.908 38.608) (end 30.48 43.18) (width 0.2) (layer "F.Cu") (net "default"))
 (segment (start 23.919728 33.971806) (end 23.368 34.523534) (width 0.2) (layer "F.Cu") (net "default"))
 (segment (start 25.599107 30.171107) (end 26.416 29.354214) (width 0.2) (layer "F.Cu") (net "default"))
 (segment (start 21.59 32.766) (end 18.034 32.766) (width 0.2) (layer "F.Cu") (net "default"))
 (segment (start 25.95266 30.43534) (end 30.48 25.908) (width 0.2) (layer "F.Cu") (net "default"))
 (segment (start 26.659767 32.204039) (end 27.475728 33.02) (width 0.2) (layer "F.Cu") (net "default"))
 (segment (start 26.416 34.081592) (end 26.416 36.576) (width 0.2) (layer "F.Cu") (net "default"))
 (segment (start 22.151961 31.231767) (end 21.654194 30.734) (width 0.2) (layer "F.Cu") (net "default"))
 (segment (start 23.212621 30.171107) (end 22.352 29.310486) (width 0.2) (layer "F.Cu") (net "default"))
 (segment (start 22.86 25.4) (end 17.78 20.32) (width 0.2) (layer "F.Cu") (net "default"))
 (segment (start 22.505515 32.557592) (end 19.503108 35.56) (width 0.2) (layer "F.Cu") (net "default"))
 (segment (start 22.86 29.111379) (end 22.86 25.4) (width 0.2) (layer "F.Cu") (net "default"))
 (segment (start 26.659767 31.231767) (end 27.411534 30.48) (width 0.2) (layer "F.Cu") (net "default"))
 (segment (start 24.892 33.971806) (end 25.4 34.479806) (width 0.2) (layer "F.Cu") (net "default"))
 (segment (start 23.368 23.368) (end 17.78 17.78) (width 0.2) (layer "F.Cu") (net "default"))
 (segment (start 26.306213 32.656213) (end 29.21 35.56) (width 0.2) (layer "F.Cu") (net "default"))
 (segment (start 23.368 34.523534) (end 23.368 40.132) (width 0.2) (layer "F.Cu") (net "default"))
 (segment (start 25.908 29.155107) (end 25.908 24.891999) (width 0.2) (layer "F.Cu") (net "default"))
 (segment (start 26.416 26.924) (end 30.48 22.86) (width 0.2) (layer "F.Cu") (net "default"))
 (segment (start 26.416 36.576) (end 30.48 40.64) (width 0.2) (layer "F.Cu") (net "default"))
 (segment (start 24.892 29.464) (end 25.4 28.956) (width 0.2) (layer "F.Cu") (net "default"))
 (segment (start 23.919728 29.464) (end 23.368 28.912272) (width 0.2) (layer "F.Cu") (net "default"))
 (segment (start 25.95266 33.06466) (end 30.48 37.592) (width 0.2) (layer "F.Cu") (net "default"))
 (segment (start 25.4 34.479806) (end 25.4 40.64) (width 0.2) (layer "F.Cu") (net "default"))
 (segment (start 23.566175 29.817554) (end 22.86 29.111379) (width 0.2) (layer "F.Cu") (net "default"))
 (segment (start 25.4 28.956) (end 25.4 22.86) (width 0.2) (layer "F.Cu") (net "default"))
 (segment (start 25.4 40.64) (end 30.48 45.72) (width 0.2) (layer "F.Cu") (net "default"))
 (segment (start 22.86 38.1) (end 17.78 43.18) (width 0.2) (layer "F.Cu") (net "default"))
 (segment (start 21.654194 30.734) (end 18.034 30.734) (width 0.2) (layer "F.Cu") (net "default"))
 (segment (start 30.48 37.592) (end 30.48 38.1) (width 0.2) (layer "F.Cu") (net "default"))
 (segment (start 27.411534 30.48) (end 30.48 30.48) (width 0.2) (layer "F.Cu") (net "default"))
 (segment (start 30.353 38.1) (end 30.48 38.1) (width 0.2) (layer "F.Cu") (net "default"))
 (segment (start 23.212621 33.264699) (end 22.352 34.12532) (width 0.2) (layer "F.Cu") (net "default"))
 (segment (start 22.859068 32.911146) (end 22.859068 33.020932) (width 0.2) (layer "F.Cu") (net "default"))
 (segment (start 25.95266 30.52466) (end 25.95266 30.43534) (width 0.2) (layer "F.Cu") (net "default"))
 (segment (start 22.352 29.310486) (end 22.352 27.432) (width 0.2) (layer "F.Cu") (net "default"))
 (segment (start 23.368 28.912272) (end 23.368 23.368) (width 0.2) (layer "F.Cu") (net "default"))
 (segment (start 29.21 35.56) (end 30.48 35.56) (width 0.2) (layer "F.Cu") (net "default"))
 (segment (start 25.245553 29.817554) (end 25.908 29.155107) (width 0.2) (layer "F.Cu") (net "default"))
 (segment (start 21.59 31.75) (end 24.384 31.75) (width 0.2) (layer "B.Cu") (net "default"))
 (segment (start 17.78 35.56) (end 21.59 31.75) (width 0.2) (layer "B.Cu") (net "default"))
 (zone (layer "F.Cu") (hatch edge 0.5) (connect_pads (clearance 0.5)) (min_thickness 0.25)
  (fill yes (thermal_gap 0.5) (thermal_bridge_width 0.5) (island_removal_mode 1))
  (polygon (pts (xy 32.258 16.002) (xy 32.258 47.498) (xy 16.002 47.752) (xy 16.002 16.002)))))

